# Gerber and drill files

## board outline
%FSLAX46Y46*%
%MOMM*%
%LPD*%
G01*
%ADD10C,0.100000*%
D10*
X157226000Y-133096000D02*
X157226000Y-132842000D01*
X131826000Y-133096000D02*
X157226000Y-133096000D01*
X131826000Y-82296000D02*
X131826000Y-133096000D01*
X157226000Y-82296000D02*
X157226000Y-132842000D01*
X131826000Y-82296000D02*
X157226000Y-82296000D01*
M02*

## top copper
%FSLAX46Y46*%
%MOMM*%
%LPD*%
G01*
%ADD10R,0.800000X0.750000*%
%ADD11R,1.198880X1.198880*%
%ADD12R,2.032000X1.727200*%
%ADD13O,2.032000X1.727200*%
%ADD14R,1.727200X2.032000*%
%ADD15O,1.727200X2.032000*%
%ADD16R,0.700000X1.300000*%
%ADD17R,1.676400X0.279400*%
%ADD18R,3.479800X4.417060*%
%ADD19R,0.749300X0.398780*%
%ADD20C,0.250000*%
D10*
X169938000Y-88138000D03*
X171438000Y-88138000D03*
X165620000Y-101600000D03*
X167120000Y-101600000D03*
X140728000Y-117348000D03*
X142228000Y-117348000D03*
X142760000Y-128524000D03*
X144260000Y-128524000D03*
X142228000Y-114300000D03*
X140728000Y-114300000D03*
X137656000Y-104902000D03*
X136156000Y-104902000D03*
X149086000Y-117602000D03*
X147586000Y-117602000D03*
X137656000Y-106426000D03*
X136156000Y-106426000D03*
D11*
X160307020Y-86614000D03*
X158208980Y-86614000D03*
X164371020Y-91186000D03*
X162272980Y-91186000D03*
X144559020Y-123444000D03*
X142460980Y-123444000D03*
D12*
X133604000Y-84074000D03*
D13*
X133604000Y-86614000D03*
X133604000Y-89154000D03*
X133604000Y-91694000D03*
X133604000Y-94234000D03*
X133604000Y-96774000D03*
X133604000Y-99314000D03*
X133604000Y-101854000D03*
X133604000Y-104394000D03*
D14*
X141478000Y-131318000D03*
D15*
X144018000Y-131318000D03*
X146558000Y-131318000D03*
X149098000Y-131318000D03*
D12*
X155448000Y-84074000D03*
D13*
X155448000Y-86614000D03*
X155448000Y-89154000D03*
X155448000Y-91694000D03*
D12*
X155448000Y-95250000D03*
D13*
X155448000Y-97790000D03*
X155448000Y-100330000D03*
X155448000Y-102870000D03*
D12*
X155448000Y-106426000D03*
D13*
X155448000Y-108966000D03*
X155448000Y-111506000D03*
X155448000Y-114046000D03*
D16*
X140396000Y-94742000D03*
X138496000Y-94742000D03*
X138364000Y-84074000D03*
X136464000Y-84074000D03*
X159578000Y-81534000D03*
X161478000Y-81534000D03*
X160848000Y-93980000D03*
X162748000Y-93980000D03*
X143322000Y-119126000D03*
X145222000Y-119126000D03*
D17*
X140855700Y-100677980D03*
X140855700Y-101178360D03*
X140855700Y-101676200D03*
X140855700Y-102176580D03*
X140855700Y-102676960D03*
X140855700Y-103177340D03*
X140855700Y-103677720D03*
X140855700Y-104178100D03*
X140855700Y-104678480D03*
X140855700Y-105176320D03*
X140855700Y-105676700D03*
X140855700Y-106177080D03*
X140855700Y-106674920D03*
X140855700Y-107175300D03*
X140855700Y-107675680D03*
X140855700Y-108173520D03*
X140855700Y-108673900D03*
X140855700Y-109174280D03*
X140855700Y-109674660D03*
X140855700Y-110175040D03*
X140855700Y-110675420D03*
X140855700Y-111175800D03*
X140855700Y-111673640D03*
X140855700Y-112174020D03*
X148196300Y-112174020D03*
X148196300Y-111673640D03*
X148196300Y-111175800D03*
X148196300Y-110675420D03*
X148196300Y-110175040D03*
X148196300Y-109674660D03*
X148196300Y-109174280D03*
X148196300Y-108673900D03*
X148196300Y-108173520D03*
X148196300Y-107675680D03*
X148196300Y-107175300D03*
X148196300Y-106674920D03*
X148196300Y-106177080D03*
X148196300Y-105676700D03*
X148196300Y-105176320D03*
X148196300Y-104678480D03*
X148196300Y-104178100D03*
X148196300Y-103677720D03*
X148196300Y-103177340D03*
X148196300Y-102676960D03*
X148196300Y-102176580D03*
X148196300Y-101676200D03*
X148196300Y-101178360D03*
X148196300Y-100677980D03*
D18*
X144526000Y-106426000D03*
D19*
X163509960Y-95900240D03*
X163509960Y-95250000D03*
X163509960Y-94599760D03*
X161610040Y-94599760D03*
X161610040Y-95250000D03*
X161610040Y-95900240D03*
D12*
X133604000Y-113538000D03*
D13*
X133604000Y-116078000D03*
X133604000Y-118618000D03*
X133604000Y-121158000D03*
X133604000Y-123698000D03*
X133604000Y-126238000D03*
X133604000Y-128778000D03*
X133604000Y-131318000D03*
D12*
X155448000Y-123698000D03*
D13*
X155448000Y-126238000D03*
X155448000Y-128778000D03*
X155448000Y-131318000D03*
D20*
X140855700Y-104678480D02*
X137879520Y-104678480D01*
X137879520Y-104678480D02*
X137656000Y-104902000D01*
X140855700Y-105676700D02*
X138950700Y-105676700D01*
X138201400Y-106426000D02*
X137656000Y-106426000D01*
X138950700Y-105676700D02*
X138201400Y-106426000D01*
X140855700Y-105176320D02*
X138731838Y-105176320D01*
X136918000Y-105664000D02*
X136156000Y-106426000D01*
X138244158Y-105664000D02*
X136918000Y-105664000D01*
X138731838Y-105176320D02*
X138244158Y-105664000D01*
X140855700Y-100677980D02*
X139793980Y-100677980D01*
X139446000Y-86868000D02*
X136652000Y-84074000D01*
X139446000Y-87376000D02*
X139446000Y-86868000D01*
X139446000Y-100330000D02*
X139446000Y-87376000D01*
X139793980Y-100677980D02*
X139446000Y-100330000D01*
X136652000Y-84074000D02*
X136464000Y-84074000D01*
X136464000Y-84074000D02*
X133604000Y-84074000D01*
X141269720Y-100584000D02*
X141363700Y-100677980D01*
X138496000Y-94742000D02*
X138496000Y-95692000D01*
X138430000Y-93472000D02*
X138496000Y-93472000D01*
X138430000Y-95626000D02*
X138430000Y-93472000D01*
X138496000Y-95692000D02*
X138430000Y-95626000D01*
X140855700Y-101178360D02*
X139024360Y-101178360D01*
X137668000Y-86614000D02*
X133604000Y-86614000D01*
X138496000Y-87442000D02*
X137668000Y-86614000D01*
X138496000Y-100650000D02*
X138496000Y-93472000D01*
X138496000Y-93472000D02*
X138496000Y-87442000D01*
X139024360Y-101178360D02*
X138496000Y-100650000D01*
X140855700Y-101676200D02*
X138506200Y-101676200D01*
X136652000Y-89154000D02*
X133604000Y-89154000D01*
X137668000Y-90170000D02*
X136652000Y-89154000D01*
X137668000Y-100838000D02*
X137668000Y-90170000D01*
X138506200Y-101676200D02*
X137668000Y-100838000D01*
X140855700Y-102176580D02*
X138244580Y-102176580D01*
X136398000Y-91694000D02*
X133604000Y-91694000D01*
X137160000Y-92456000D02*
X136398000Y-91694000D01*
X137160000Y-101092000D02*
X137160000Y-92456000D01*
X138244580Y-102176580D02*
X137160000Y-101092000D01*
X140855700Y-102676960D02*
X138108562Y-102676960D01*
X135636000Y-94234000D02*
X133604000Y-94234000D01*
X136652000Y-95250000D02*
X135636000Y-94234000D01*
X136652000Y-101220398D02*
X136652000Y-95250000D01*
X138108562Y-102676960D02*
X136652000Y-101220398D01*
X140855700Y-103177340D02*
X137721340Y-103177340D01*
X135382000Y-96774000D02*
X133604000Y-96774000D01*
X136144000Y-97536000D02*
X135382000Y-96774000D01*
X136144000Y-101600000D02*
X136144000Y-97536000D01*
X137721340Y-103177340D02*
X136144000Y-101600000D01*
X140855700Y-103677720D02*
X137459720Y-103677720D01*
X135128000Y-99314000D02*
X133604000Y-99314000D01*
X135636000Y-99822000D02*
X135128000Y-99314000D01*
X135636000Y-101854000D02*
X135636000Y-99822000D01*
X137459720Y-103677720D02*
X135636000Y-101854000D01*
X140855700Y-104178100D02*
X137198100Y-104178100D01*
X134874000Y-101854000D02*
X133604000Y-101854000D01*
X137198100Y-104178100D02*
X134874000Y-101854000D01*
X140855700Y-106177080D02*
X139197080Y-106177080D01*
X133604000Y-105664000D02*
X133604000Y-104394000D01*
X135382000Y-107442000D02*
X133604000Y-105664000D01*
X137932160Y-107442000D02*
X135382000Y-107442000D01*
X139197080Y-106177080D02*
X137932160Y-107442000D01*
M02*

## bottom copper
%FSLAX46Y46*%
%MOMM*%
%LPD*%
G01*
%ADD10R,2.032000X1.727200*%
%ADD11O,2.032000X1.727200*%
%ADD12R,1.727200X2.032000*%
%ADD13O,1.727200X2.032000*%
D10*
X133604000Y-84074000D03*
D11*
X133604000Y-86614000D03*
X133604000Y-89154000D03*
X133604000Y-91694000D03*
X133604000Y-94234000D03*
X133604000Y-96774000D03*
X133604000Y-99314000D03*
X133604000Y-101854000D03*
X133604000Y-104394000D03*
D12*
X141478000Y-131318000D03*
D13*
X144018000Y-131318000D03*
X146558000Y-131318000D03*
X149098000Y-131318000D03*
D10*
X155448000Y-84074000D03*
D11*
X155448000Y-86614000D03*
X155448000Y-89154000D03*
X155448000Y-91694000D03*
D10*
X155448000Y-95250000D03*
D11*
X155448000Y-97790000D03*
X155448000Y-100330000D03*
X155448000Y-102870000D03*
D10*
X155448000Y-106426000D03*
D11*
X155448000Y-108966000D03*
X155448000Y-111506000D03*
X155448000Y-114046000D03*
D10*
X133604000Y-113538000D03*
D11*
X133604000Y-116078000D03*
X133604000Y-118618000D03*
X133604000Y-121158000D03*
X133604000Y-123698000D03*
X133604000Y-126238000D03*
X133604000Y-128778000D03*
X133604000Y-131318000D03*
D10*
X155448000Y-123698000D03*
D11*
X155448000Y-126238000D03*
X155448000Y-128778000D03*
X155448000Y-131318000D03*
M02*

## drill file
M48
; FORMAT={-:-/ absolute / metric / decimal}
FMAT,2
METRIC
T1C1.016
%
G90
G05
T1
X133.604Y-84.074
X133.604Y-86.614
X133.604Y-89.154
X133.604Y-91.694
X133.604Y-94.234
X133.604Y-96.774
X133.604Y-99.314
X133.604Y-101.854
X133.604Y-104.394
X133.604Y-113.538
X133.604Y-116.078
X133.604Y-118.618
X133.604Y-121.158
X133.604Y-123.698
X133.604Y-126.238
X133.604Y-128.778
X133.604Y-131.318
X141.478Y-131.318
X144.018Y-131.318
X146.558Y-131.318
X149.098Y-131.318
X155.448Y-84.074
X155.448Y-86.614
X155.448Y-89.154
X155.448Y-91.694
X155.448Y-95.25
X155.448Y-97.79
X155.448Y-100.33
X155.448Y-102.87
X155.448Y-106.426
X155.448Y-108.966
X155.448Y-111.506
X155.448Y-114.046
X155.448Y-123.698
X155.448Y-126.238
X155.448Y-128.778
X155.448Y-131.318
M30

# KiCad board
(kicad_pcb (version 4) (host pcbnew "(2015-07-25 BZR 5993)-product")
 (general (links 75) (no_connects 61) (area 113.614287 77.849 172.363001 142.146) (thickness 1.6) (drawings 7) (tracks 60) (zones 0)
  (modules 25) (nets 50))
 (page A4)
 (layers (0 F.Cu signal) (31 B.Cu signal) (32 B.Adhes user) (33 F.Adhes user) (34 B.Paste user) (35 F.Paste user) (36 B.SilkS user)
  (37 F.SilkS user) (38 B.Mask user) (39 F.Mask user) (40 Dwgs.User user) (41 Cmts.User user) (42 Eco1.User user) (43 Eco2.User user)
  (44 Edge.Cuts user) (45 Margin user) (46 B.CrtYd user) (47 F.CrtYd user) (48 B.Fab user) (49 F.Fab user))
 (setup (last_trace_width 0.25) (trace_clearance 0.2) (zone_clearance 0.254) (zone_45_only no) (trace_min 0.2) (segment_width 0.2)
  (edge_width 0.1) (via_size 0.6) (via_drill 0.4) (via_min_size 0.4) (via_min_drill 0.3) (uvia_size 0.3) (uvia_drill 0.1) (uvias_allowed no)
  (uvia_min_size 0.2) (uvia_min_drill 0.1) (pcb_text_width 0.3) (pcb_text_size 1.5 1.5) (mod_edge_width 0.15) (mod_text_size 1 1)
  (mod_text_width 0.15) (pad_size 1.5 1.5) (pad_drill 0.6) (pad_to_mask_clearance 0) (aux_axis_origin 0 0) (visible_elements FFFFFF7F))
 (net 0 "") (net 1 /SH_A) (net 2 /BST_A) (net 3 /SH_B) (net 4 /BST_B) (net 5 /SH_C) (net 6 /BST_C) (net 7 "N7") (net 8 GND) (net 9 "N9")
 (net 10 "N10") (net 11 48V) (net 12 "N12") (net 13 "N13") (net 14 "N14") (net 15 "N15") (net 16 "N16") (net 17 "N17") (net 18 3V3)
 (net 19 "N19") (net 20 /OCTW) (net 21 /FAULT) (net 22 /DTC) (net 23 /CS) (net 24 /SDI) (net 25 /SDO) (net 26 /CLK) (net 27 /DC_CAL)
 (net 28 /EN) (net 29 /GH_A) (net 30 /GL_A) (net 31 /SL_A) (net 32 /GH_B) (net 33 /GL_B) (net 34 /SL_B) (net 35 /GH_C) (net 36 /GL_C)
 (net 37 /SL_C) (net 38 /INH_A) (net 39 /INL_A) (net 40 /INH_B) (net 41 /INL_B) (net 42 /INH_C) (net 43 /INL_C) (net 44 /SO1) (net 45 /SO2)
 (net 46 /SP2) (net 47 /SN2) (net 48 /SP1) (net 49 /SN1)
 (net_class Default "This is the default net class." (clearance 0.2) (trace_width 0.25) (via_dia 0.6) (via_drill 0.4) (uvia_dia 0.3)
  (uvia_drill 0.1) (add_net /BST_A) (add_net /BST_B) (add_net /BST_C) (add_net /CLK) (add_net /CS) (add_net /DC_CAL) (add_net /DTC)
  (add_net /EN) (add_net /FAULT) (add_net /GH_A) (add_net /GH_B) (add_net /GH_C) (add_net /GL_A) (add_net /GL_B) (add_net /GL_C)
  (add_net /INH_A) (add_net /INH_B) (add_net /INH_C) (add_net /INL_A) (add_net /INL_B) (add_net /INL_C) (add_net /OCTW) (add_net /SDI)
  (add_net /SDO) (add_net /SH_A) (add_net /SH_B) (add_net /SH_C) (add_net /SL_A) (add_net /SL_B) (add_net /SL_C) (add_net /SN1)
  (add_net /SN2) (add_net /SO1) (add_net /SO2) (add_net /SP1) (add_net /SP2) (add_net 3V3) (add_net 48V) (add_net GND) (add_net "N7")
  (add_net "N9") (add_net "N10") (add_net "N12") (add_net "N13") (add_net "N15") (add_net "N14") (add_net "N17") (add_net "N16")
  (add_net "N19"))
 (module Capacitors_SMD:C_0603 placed (layer F.Cu) (at 170.688 88.138)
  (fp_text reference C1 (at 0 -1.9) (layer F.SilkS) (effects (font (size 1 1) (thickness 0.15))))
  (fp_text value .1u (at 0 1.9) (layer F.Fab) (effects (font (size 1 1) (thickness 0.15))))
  (pad 1 smd rect (at -0.75 0) (size 0.8 0.75) (layers F.Cu F.Paste F.Mask) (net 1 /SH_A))
  (pad 2 smd rect (at 0.75 0) (size 0.8 0.75) (layers F.Cu F.Paste F.Mask) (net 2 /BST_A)))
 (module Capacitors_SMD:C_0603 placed (layer F.Cu) (at 166.37 101.6)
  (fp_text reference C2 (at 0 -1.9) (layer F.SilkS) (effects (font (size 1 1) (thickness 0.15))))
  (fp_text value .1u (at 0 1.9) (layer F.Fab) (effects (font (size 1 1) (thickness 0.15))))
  (pad 1 smd rect (at -0.75 0) (size 0.8 0.75) (layers F.Cu F.Paste F.Mask) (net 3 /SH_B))
  (pad 2 smd rect (at 0.75 0) (size 0.8 0.75) (layers F.Cu F.Paste F.Mask) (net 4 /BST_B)))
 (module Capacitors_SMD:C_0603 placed (layer F.Cu) (at 141.478 117.348)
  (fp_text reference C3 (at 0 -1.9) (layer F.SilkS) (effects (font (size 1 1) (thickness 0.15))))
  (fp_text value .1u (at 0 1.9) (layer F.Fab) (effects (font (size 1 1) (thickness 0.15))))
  (pad 1 smd rect (at -0.75 0) (size 0.8 0.75) (layers F.Cu F.Paste F.Mask) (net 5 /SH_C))
  (pad 2 smd rect (at 0.75 0) (size 0.8 0.75) (layers F.Cu F.Paste F.Mask) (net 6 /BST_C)))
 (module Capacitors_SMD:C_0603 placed (layer F.Cu) (at 143.51 128.524)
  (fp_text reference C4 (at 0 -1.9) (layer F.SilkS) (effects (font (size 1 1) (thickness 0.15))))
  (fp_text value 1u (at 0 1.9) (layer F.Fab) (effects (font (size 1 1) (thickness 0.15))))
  (pad 1 smd rect (at -0.75 0) (size 0.8 0.75) (layers F.Cu F.Paste F.Mask) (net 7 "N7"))
  (pad 2 smd rect (at 0.75 0) (size 0.8 0.75) (layers F.Cu F.Paste F.Mask) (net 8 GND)))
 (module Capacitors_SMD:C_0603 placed (layer F.Cu) (at 141.478 114.3 180)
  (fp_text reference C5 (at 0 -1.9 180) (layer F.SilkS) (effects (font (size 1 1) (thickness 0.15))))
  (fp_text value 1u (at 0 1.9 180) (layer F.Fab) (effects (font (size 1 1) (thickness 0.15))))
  (pad 1 smd rect (at -0.75 0 180) (size 0.8 0.75) (layers F.Cu F.Paste F.Mask) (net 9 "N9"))
  (pad 2 smd rect (at 0.75 0 180) (size 0.8 0.75) (layers F.Cu F.Paste F.Mask) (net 8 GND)))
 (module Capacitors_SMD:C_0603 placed (layer F.Cu) (at 136.906 104.902 180)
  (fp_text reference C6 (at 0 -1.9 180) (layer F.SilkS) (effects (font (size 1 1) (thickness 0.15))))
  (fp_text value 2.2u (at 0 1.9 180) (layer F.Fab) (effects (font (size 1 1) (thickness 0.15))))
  (pad 1 smd rect (at -0.75 0 180) (size 0.8 0.75) (layers F.Cu F.Paste F.Mask) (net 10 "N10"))
  (pad 2 smd rect (at 0.75 0 180) (size 0.8 0.75) (layers F.Cu F.Paste F.Mask) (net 8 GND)))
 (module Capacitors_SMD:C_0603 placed (layer F.Cu) (at 148.336 117.602 180)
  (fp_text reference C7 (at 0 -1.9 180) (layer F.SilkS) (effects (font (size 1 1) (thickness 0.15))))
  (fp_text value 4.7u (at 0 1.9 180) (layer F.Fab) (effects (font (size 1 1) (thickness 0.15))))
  (pad 1 smd rect (at -0.75 0 180) (size 0.8 0.75) (layers F.Cu F.Paste F.Mask) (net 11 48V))
  (pad 2 smd rect (at 0.75 0 180) (size 0.8 0.75) (layers F.Cu F.Paste F.Mask) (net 8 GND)))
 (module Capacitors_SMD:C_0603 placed (layer F.Cu) (at 136.906 106.426 180)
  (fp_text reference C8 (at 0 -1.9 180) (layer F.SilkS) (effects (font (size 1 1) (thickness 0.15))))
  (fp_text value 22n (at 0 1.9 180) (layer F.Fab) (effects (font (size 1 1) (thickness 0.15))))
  (pad 1 smd rect (at -0.75 0 180) (size 0.8 0.75) (layers F.Cu F.Paste F.Mask) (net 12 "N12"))
  (pad 2 smd rect (at 0.75 0 180) (size 0.8 0.75) (layers F.Cu F.Paste F.Mask) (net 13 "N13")))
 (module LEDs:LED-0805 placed (layer F.Cu) (at 159.258 86.614)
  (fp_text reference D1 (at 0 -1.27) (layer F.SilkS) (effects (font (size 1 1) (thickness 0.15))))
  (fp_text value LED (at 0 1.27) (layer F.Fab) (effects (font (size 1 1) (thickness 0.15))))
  (pad 2 smd rect (at 1.04902 0 180) (size 1.19888 1.19888) (layers F.Cu F.Paste F.Mask) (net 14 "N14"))
  (pad 1 smd rect (at -1.04902 0 180) (size 1.19888 1.19888) (layers F.Cu F.Paste F.Mask) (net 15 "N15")))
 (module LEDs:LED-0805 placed (layer F.Cu) (at 163.322 91.186)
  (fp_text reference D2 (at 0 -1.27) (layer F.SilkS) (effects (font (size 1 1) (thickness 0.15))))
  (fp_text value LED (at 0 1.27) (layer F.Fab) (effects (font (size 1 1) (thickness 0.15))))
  (pad 2 smd rect (at 1.04902 0 180) (size 1.19888 1.19888) (layers F.Cu F.Paste F.Mask) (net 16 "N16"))
  (pad 1 smd rect (at -1.04902 0 180) (size 1.19888 1.19888) (layers F.Cu F.Paste F.Mask) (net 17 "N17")))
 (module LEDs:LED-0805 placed (layer F.Cu) (at 143.51 123.444)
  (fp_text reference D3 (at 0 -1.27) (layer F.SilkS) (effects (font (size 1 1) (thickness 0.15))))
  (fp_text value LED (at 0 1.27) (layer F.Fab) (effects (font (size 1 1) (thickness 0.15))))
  (pad 2 smd rect (at 1.04902 0 180) (size 1.19888 1.19888) (layers F.Cu F.Paste F.Mask) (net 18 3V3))
  (pad 1 smd rect (at -1.04902 0 180) (size 1.19888 1.19888) (layers F.Cu F.Paste F.Mask) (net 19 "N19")))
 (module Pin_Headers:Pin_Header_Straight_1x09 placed (layer F.Cu) (at 133.604 84.074)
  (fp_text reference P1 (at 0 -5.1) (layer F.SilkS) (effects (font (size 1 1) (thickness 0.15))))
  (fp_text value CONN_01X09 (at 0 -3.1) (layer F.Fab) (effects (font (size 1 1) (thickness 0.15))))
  (pad 1 thru_hole rect (at 0 0) (size 2.032 1.7272) (drill 1.016) (layers *.Cu *.Mask F.SilkS) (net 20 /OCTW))
  (pad 2 thru_hole oval (at 0 2.54) (size 2.032 1.7272) (drill 1.016) (layers *.Cu *.Mask F.SilkS) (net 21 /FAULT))
  (pad 3 thru_hole oval (at 0 5.08) (size 2.032 1.7272) (drill 1.016) (layers *.Cu *.Mask F.SilkS) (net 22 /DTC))
  (pad 4 thru_hole oval (at 0 7.62) (size 2.032 1.7272) (drill 1.016) (layers *.Cu *.Mask F.SilkS) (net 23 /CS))
  (pad 5 thru_hole oval (at 0 10.16) (size 2.032 1.7272) (drill 1.016) (layers *.Cu *.Mask F.SilkS) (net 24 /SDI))
  (pad 6 thru_hole oval (at 0 12.7) (size 2.032 1.7272) (drill 1.016) (layers *.Cu *.Mask F.SilkS) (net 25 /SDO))
  (pad 7 thru_hole oval (at 0 15.24) (size 2.032 1.7272) (drill 1.016) (layers *.Cu *.Mask F.SilkS) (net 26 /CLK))
  (pad 8 thru_hole oval (at 0 17.78) (size 2.032 1.7272) (drill 1.016) (layers *.Cu *.Mask F.SilkS) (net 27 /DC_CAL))
  (pad 9 thru_hole oval (at 0 20.32) (size 2.032 1.7272) (drill 1.016) (layers *.Cu *.Mask F.SilkS) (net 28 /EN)))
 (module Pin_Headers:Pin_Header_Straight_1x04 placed (layer F.Cu) (at 141.478 131.318 90)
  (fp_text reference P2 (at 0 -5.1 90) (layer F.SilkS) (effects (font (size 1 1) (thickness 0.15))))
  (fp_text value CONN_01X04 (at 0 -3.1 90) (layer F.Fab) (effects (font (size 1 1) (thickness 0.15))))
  (pad 1 thru_hole rect (at 0 0 90) (size 2.032 1.7272) (drill 1.016) (layers *.Cu *.Mask F.SilkS) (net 18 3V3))
  (pad 2 thru_hole oval (at 0 2.54 90) (size 2.032 1.7272) (drill 1.016) (layers *.Cu *.Mask F.SilkS) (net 11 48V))
  (pad 3 thru_hole oval (at 0 5.08 90) (size 2.032 1.7272) (drill 1.016) (layers *.Cu *.Mask F.SilkS) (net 8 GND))
  (pad 4 thru_hole oval (at 0 7.62 90) (size 2.032 1.7272) (drill 1.016) (layers *.Cu *.Mask F.SilkS) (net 8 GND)))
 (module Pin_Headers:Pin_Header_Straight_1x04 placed (layer F.Cu) (at 155.448 84.074)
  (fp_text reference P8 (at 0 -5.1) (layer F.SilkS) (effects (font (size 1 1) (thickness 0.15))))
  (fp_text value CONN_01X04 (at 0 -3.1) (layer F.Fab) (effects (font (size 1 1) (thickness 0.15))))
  (pad 1 thru_hole rect (at 0 0) (size 2.032 1.7272) (drill 1.016) (layers *.Cu *.Mask F.SilkS) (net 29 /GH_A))
  (pad 2 thru_hole oval (at 0 2.54) (size 2.032 1.7272) (drill 1.016) (layers *.Cu *.Mask F.SilkS) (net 1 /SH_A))
  (pad 3 thru_hole oval (at 0 5.08) (size 2.032 1.7272) (drill 1.016) (layers *.Cu *.Mask F.SilkS) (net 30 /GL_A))
  (pad 4 thru_hole oval (at 0 7.62) (size 2.032 1.7272) (drill 1.016) (layers *.Cu *.Mask F.SilkS) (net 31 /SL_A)))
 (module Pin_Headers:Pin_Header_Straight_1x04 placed (layer F.Cu) (at 155.448 95.25)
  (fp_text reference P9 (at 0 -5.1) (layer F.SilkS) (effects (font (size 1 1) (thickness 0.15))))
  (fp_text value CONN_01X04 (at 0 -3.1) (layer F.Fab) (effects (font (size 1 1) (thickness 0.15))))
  (pad 1 thru_hole rect (at 0 0) (size 2.032 1.7272) (drill 1.016) (layers *.Cu *.Mask F.SilkS) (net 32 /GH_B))
  (pad 2 thru_hole oval (at 0 2.54) (size 2.032 1.7272) (drill 1.016) (layers *.Cu *.Mask F.SilkS) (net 3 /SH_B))
  (pad 3 thru_hole oval (at 0 5.08) (size 2.032 1.7272) (drill 1.016) (layers *.Cu *.Mask F.SilkS) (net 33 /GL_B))
  (pad 4 thru_hole oval (at 0 7.62) (size 2.032 1.7272) (drill 1.016) (layers *.Cu *.Mask F.SilkS) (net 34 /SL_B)))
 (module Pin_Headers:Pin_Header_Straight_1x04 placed (layer F.Cu) (at 155.448 106.426)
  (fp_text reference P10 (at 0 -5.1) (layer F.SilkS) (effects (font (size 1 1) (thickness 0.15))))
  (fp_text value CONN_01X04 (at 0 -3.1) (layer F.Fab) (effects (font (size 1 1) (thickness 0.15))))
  (pad 1 thru_hole rect (at 0 0) (size 2.032 1.7272) (drill 1.016) (layers *.Cu *.Mask F.SilkS) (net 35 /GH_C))
  (pad 2 thru_hole oval (at 0 2.54) (size 2.032 1.7272) (drill 1.016) (layers *.Cu *.Mask F.SilkS) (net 5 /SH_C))
  (pad 3 thru_hole oval (at 0 5.08) (size 2.032 1.7272) (drill 1.016) (layers *.Cu *.Mask F.SilkS) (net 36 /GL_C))
  (pad 4 thru_hole oval (at 0 7.62) (size 2.032 1.7272) (drill 1.016) (layers *.Cu *.Mask F.SilkS) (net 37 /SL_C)))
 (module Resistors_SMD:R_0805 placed (layer F.Cu) (at 139.446 94.742 180)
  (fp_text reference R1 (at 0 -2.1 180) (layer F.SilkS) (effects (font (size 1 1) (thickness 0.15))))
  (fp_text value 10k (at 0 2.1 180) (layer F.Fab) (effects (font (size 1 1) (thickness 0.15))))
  (pad 1 smd rect (at -0.95 0 180) (size 0.7 1.3) (layers F.Cu F.Paste F.Mask) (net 18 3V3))
  (pad 2 smd rect (at 0.95 0 180) (size 0.7 1.3) (layers F.Cu F.Paste F.Mask) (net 21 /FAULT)))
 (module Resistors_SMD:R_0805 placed (layer F.Cu) (at 137.414 84.074 180)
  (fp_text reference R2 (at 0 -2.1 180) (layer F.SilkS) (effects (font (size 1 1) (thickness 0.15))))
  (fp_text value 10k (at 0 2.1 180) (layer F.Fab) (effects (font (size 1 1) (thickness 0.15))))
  (pad 1 smd rect (at -0.95 0 180) (size 0.7 1.3) (layers F.Cu F.Paste F.Mask) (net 18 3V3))
  (pad 2 smd rect (at 0.95 0 180) (size 0.7 1.3) (layers F.Cu F.Paste F.Mask) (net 20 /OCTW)))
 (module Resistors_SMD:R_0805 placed (layer F.Cu) (at 160.528 81.534)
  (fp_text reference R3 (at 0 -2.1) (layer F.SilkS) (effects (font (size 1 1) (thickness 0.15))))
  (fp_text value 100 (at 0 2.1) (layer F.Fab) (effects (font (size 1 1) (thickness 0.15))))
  (pad 1 smd rect (at -0.95 0) (size 0.7 1.3) (layers F.Cu F.Paste F.Mask) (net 15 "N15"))
  (pad 2 smd rect (at 0.95 0) (size 0.7 1.3) (layers F.Cu F.Paste F.Mask) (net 8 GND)))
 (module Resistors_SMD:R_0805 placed (layer F.Cu) (at 161.798 93.98)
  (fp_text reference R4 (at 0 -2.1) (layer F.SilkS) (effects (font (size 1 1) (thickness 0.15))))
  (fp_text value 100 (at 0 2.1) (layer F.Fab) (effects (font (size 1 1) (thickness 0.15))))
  (pad 1 smd rect (at -0.95 0) (size 0.7 1.3) (layers F.Cu F.Paste F.Mask) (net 17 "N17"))
  (pad 2 smd rect (at 0.95 0) (size 0.7 1.3) (layers F.Cu F.Paste F.Mask) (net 8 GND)))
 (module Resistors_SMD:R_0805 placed (layer F.Cu) (at 144.272 119.126)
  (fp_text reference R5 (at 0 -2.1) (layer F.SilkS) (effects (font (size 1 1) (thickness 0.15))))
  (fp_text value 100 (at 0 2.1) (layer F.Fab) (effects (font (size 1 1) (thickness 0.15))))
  (pad 1 smd rect (at -0.95 0) (size 0.7 1.3) (layers F.Cu F.Paste F.Mask) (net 19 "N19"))
  (pad 2 smd rect (at 0.95 0) (size 0.7 1.3) (layers F.Cu F.Paste F.Mask) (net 8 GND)))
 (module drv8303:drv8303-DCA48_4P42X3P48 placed (layer F.Cu) (at 144.526 106.426)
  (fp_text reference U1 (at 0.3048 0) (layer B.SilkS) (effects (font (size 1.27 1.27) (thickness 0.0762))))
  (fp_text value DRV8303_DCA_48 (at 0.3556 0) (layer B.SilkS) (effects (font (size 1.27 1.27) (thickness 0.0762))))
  (pad 1 smd rect (at -3.6703 -5.74802) (size 1.6764 0.2794) (layers F.Cu F.Paste F.Mask) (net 20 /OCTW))
  (pad 2 smd rect (at -3.6703 -5.24764) (size 1.6764 0.2794) (layers F.Cu F.Paste F.Mask) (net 21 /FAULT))
  (pad 3 smd rect (at -3.6703 -4.7498) (size 1.6764 0.2794) (layers F.Cu F.Paste F.Mask) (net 22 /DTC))
  (pad 4 smd rect (at -3.6703 -4.24942) (size 1.6764 0.2794) (layers F.Cu F.Paste F.Mask) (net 23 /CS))
  (pad 5 smd rect (at -3.6703 -3.74904) (size 1.6764 0.2794) (layers F.Cu F.Paste F.Mask) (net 24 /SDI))
  (pad 6 smd rect (at -3.6703 -3.24866) (size 1.6764 0.2794) (layers F.Cu F.Paste F.Mask) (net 25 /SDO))
  (pad 7 smd rect (at -3.6703 -2.74828) (size 1.6764 0.2794) (layers F.Cu F.Paste F.Mask) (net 26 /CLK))
  (pad 8 smd rect (at -3.6703 -2.2479) (size 1.6764 0.2794) (layers F.Cu F.Paste F.Mask) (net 27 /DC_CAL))
  (pad 9 smd rect (at -3.6703 -1.74752) (size 1.6764 0.2794) (layers F.Cu F.Paste F.Mask) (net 10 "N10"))
  (pad 10 smd rect (at -3.6703 -1.24968) (size 1.6764 0.2794) (layers F.Cu F.Paste F.Mask) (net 13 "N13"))
  (pad 11 smd rect (at -3.6703 -0.7493) (size 1.6764 0.2794) (layers F.Cu F.Paste F.Mask) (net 12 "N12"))
  (pad 12 smd rect (at -3.6703 -0.24892) (size 1.6764 0.2794) (layers F.Cu F.Paste F.Mask) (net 28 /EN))
  (pad 13 smd rect (at -3.6703 0.24892) (size 1.6764 0.2794) (layers F.Cu F.Paste F.Mask) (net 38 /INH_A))
  (pad 14 smd rect (at -3.6703 0.7493) (size 1.6764 0.2794) (layers F.Cu F.Paste F.Mask) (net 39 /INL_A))
  (pad 15 smd rect (at -3.6703 1.24968) (size 1.6764 0.2794) (layers F.Cu F.Paste F.Mask) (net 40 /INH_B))
  (pad 16 smd rect (at -3.6703 1.74752) (size 1.6764 0.2794) (layers F.Cu F.Paste F.Mask) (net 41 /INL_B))
  (pad 17 smd rect (at -3.6703 2.2479) (size 1.6764 0.2794) (layers F.Cu F.Paste F.Mask) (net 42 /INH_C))
  (pad 18 smd rect (at -3.6703 2.74828) (size 1.6764 0.2794) (layers F.Cu F.Paste F.Mask) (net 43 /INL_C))
  (pad 19 smd rect (at -3.6703 3.24866) (size 1.6764 0.2794) (layers F.Cu F.Paste F.Mask) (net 9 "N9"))
  (pad 20 smd rect (at -3.6703 3.74904) (size 1.6764 0.2794) (layers F.Cu F.Paste F.Mask) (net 18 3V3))
  (pad 21 smd rect (at -3.6703 4.24942) (size 1.6764 0.2794) (layers F.Cu F.Paste F.Mask) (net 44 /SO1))
  (pad 22 smd rect (at -3.6703 4.7498) (size 1.6764 0.2794) (layers F.Cu F.Paste F.Mask) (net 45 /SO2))
  (pad 23 smd rect (at -3.6703 5.24764) (size 1.6764 0.2794) (layers F.Cu F.Paste F.Mask) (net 7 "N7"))
  (pad 24 smd rect (at -3.6703 5.74802) (size 1.6764 0.2794) (layers F.Cu F.Paste F.Mask) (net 8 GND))
  (pad 25 smd rect (at 3.6703 5.74802) (size 1.6764 0.2794) (layers F.Cu F.Paste F.Mask) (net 11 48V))
  (pad 26 smd rect (at 3.6703 5.24764) (size 1.6764 0.2794) (layers F.Cu F.Paste F.Mask) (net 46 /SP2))
  (pad 27 smd rect (at 3.6703 4.7498) (size 1.6764 0.2794) (layers F.Cu F.Paste F.Mask) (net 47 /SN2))
  (pad 28 smd rect (at 3.6703 4.24942) (size 1.6764 0.2794) (layers F.Cu F.Paste F.Mask) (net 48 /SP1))
  (pad 29 smd rect (at 3.6703 3.74904) (size 1.6764 0.2794) (layers F.Cu F.Paste F.Mask) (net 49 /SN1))
  (pad 30 smd rect (at 3.6703 3.24866) (size 1.6764 0.2794) (layers F.Cu F.Paste F.Mask) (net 37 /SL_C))
  (pad 31 smd rect (at 3.6703 2.74828) (size 1.6764 0.2794) (layers F.Cu F.Paste F.Mask) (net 36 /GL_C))
  (pad 32 smd rect (at 3.6703 2.2479) (size 1.6764 0.2794) (layers F.Cu F.Paste F.Mask) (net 5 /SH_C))
  (pad 33 smd rect (at 3.6703 1.74752) (size 1.6764 0.2794) (layers F.Cu F.Paste F.Mask) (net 35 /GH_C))
  (pad 34 smd rect (at 3.6703 1.24968) (size 1.6764 0.2794) (layers F.Cu F.Paste F.Mask) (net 6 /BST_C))
  (pad 35 smd rect (at 3.6703 0.7493) (size 1.6764 0.2794) (layers F.Cu F.Paste F.Mask) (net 34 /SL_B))
  (pad 36 smd rect (at 3.6703 0.24892) (size 1.6764 0.2794) (layers F.Cu F.Paste F.Mask) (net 33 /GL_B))
  (pad 37 smd rect (at 3.6703 -0.24892) (size 1.6764 0.2794) (layers F.Cu F.Paste F.Mask) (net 3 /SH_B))
  (pad 38 smd rect (at 3.6703 -0.7493) (size 1.6764 0.2794) (layers F.Cu F.Paste F.Mask) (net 32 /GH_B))
  (pad 39 smd rect (at 3.6703 -1.24968) (size 1.6764 0.2794) (layers F.Cu F.Paste F.Mask) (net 4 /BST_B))
  (pad 40 smd rect (at 3.6703 -1.74752) (size 1.6764 0.2794) (layers F.Cu F.Paste F.Mask) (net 31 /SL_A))
  (pad 41 smd rect (at 3.6703 -2.2479) (size 1.6764 0.2794) (layers F.Cu F.Paste F.Mask) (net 30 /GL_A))
  (pad 42 smd rect (at 3.6703 -2.74828) (size 1.6764 0.2794) (layers F.Cu F.Paste F.Mask) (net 1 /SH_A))
  (pad 43 smd rect (at 3.6703 -3.24866) (size 1.6764 0.2794) (layers F.Cu F.Paste F.Mask) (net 29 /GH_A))
  (pad 44 smd rect (at 3.6703 -3.74904) (size 1.6764 0.2794) (layers F.Cu F.Paste F.Mask) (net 2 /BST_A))
  (pad 45 smd rect (at 3.6703 -4.24942) (size 1.6764 0.2794) (layers F.Cu F.Paste F.Mask) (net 18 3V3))
  (pad 46 smd rect (at 3.6703 -4.7498) (size 1.6764 0.2794) (layers F.Cu F.Paste F.Mask) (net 8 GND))
  (pad 47 smd rect (at 3.6703 -5.24764) (size 1.6764 0.2794) (layers F.Cu F.Paste F.Mask) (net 8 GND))
  (pad 48 smd rect (at 3.6703 -5.74802) (size 1.6764 0.2794) (layers F.Cu F.Paste F.Mask) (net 8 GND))
  (pad 49 smd rect (at 0 0) (size 3.4798 4.41706) (layers F.Cu F.Paste F.Mask) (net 8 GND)))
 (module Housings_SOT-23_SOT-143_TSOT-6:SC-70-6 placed (layer F.Cu) (at 162.56 95.25 90)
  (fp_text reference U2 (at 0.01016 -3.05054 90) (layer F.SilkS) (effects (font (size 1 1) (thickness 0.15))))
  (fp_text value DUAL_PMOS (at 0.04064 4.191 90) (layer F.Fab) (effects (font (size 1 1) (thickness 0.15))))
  (pad 1 smd rect (at -0.65024 0.94996 90) (size 0.39878 0.7493) (layers F.Cu F.Paste F.Mask) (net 18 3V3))
  (pad 2 smd rect (at 0 0.94996 90) (size 0.39878 0.7493) (layers F.Cu F.Paste F.Mask) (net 20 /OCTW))
  (pad 3 smd rect (at 0.65024 0.94996 90) (size 0.39878 0.7493) (layers F.Cu F.Paste F.Mask) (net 14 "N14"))
  (pad 4 smd rect (at 0.65024 -0.94996 90) (size 0.39878 0.7493) (layers F.Cu F.Paste F.Mask) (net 18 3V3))
  (pad 5 smd rect (at 0 -0.94996 90) (size 0.39878 0.7493) (layers F.Cu F.Paste F.Mask) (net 21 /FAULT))
  (pad 6 smd rect (at -0.65024 -0.94996 90) (size 0.39878 0.7493) (layers F.Cu F.Paste F.Mask) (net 16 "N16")))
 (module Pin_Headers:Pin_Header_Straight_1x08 (layer F.Cu) (at 133.604 113.538)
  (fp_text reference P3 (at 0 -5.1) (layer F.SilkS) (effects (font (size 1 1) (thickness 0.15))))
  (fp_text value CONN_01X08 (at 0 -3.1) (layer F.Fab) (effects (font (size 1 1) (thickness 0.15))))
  (pad 1 thru_hole rect (at 0 0) (size 2.032 1.7272) (drill 1.016) (layers *.Cu *.Mask F.SilkS) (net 38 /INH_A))
  (pad 2 thru_hole oval (at 0 2.54) (size 2.032 1.7272) (drill 1.016) (layers *.Cu *.Mask F.SilkS) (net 39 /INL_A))
  (pad 3 thru_hole oval (at 0 5.08) (size 2.032 1.7272) (drill 1.016) (layers *.Cu *.Mask F.SilkS) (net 40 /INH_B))
  (pad 4 thru_hole oval (at 0 7.62) (size 2.032 1.7272) (drill 1.016) (layers *.Cu *.Mask F.SilkS) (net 41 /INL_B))
  (pad 5 thru_hole oval (at 0 10.16) (size 2.032 1.7272) (drill 1.016) (layers *.Cu *.Mask F.SilkS) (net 42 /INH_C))
  (pad 6 thru_hole oval (at 0 12.7) (size 2.032 1.7272) (drill 1.016) (layers *.Cu *.Mask F.SilkS) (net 43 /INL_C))
  (pad 7 thru_hole oval (at 0 15.24) (size 2.032 1.7272) (drill 1.016) (layers *.Cu *.Mask F.SilkS) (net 44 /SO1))
  (pad 8 thru_hole oval (at 0 17.78) (size 2.032 1.7272) (drill 1.016) (layers *.Cu *.Mask F.SilkS) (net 45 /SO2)))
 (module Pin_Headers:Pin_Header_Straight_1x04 (layer F.Cu) (at 155.448 123.698)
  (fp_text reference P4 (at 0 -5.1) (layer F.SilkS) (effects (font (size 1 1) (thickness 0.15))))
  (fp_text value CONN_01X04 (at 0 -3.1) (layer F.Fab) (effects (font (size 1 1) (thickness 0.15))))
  (pad 1 thru_hole rect (at 0 0) (size 2.032 1.7272) (drill 1.016) (layers *.Cu *.Mask F.SilkS) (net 49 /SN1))
  (pad 2 thru_hole oval (at 0 2.54) (size 2.032 1.7272) (drill 1.016) (layers *.Cu *.Mask F.SilkS) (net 48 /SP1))
  (pad 3 thru_hole oval (at 0 5.08) (size 2.032 1.7272) (drill 1.016) (layers *.Cu *.Mask F.SilkS) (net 47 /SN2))
  (pad 4 thru_hole oval (at 0 7.62) (size 2.032 1.7272) (drill 1.016) (layers *.Cu *.Mask F.SilkS) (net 46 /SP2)))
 (gr_line (start 157.226 133.096) (end 157.226 132.842) (angle 90) (layer Edge.Cuts) (width 0.1))
 (gr_line (start 131.826 133.096) (end 157.226 133.096) (angle 90) (layer Edge.Cuts) (width 0.1))
 (gr_line (start 131.826 82.296) (end 131.826 133.096) (angle 90) (layer Edge.Cuts) (width 0.1))
 (gr_line (start 157.226 82.296) (end 157.226 132.842) (angle 90) (layer Edge.Cuts) (width 0.1))
 (gr_line (start 131.826 82.296) (end 157.226 82.296) (angle 90) (layer Edge.Cuts) (width 0.1))
 (segment (start 140.8557 104.67848) (end 137.87952 104.67848) (width 0.25) (layer F.Cu) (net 10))
 (segment (start 137.87952 104.67848) (end 137.656 104.902) (width 0.25) (layer F.Cu) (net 10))
 (segment (start 140.8557 105.6767) (end 138.9507 105.6767) (width 0.25) (layer F.Cu) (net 12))
 (segment (start 138.2014 106.426) (end 137.656 106.426) (width 0.25) (layer F.Cu) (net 12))
 (segment (start 138.9507 105.6767) (end 138.2014 106.426) (width 0.25) (layer F.Cu) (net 12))
 (segment (start 140.8557 105.17632) (end 138.731838 105.17632) (width 0.25) (layer F.Cu) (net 13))
 (segment (start 136.918 105.664) (end 136.156 106.426) (width 0.25) (layer F.Cu) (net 13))
 (segment (start 138.244158 105.664) (end 136.918 105.664) (width 0.25) (layer F.Cu) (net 13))
 (segment (start 138.731838 105.17632) (end 138.244158 105.664) (width 0.25) (layer F.Cu) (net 13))
 (segment (start 140.8557 100.67798) (end 139.79398 100.67798) (width 0.25) (layer F.Cu) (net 20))
 (segment (start 139.446 86.868) (end 136.652 84.074) (width 0.25) (layer F.Cu) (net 20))
 (segment (start 139.446 87.376) (end 139.446 86.868) (width 0.25) (layer F.Cu) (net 20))
 (segment (start 139.446 100.33) (end 139.446 87.376) (width 0.25) (layer F.Cu) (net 20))
 (segment (start 139.79398 100.67798) (end 139.446 100.33) (width 0.25) (layer F.Cu) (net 20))
 (segment (start 136.652 84.074) (end 136.464 84.074) (width 0.25) (layer F.Cu) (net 20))
 (segment (start 136.464 84.074) (end 133.604 84.074) (width 0.25) (layer F.Cu) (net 20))
 (segment (start 141.26972 100.584) (end 141.3637 100.67798) (width 0.25) (layer F.Cu) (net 20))
 (segment (start 138.496 94.742) (end 138.496 95.692) (width 0.25) (layer F.Cu) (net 21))
 (segment (start 138.43 93.472) (end 138.496 93.472) (width 0.25) (layer F.Cu) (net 21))
 (segment (start 138.43 95.626) (end 138.43 93.472) (width 0.25) (layer F.Cu) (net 21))
 (segment (start 138.496 95.692) (end 138.43 95.626) (width 0.25) (layer F.Cu) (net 21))
 (segment (start 140.8557 101.17836) (end 139.02436 101.17836) (width 0.25) (layer F.Cu) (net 21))
 (segment (start 137.668 86.614) (end 133.604 86.614) (width 0.25) (layer F.Cu) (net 21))
 (segment (start 138.496 87.442) (end 137.668 86.614) (width 0.25) (layer F.Cu) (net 21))
 (segment (start 138.496 100.65) (end 138.496 93.472) (width 0.25) (layer F.Cu) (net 21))
 (segment (start 138.496 93.472) (end 138.496 87.442) (width 0.25) (layer F.Cu) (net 21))
 (segment (start 139.02436 101.17836) (end 138.496 100.65) (width 0.25) (layer F.Cu) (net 21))
 (segment (start 140.8557 101.6762) (end 138.5062 101.6762) (width 0.25) (layer F.Cu) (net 22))
 (segment (start 136.652 89.154) (end 133.604 89.154) (width 0.25) (layer F.Cu) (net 22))
 (segment (start 137.668 90.17) (end 136.652 89.154) (width 0.25) (layer F.Cu) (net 22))
 (segment (start 137.668 100.838) (end 137.668 90.17) (width 0.25) (layer F.Cu) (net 22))
 (segment (start 138.5062 101.6762) (end 137.668 100.838) (width 0.25) (layer F.Cu) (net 22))
 (segment (start 140.8557 102.17658) (end 138.24458 102.17658) (width 0.25) (layer F.Cu) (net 23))
 (segment (start 136.398 91.694) (end 133.604 91.694) (width 0.25) (layer F.Cu) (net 23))
 (segment (start 137.16 92.456) (end 136.398 91.694) (width 0.25) (layer F.Cu) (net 23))
 (segment (start 137.16 101.092) (end 137.16 92.456) (width 0.25) (layer F.Cu) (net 23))
 (segment (start 138.24458 102.17658) (end 137.16 101.092) (width 0.25) (layer F.Cu) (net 23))
 (segment (start 140.8557 102.67696) (end 138.108562 102.67696) (width 0.25) (layer F.Cu) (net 24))
 (segment (start 135.636 94.234) (end 133.604 94.234) (width 0.25) (layer F.Cu) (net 24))
 (segment (start 136.652 95.25) (end 135.636 94.234) (width 0.25) (layer F.Cu) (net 24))
 (segment (start 136.652 101.220398) (end 136.652 95.25) (width 0.25) (layer F.Cu) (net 24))
 (segment (start 138.108562 102.67696) (end 136.652 101.220398) (width 0.25) (layer F.Cu) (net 24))
 (segment (start 140.8557 103.17734) (end 137.72134 103.17734) (width 0.25) (layer F.Cu) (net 25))
 (segment (start 135.382 96.774) (end 133.604 96.774) (width 0.25) (layer F.Cu) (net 25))
 (segment (start 136.144 97.536) (end 135.382 96.774) (width 0.25) (layer F.Cu) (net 25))
 (segment (start 136.144 101.6) (end 136.144 97.536) (width 0.25) (layer F.Cu) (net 25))
 (segment (start 137.72134 103.17734) (end 136.144 101.6) (width 0.25) (layer F.Cu) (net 25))
 (segment (start 140.8557 103.67772) (end 137.45972 103.67772) (width 0.25) (layer F.Cu) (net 26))
 (segment (start 135.128 99.314) (end 133.604 99.314) (width 0.25) (layer F.Cu) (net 26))
 (segment (start 135.636 99.822) (end 135.128 99.314) (width 0.25) (layer F.Cu) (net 26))
 (segment (start 135.636 101.854) (end 135.636 99.822) (width 0.25) (layer F.Cu) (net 26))
 (segment (start 137.45972 103.67772) (end 135.636 101.854) (width 0.25) (layer F.Cu) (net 26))
 (segment (start 140.8557 104.1781) (end 137.1981 104.1781) (width 0.25) (layer F.Cu) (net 27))
 (segment (start 134.874 101.854) (end 133.604 101.854) (width 0.25) (layer F.Cu) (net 27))
 (segment (start 137.1981 104.1781) (end 134.874 101.854) (width 0.25) (layer F.Cu) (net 27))
 (segment (start 140.8557 106.17708) (end 139.19708 106.17708) (width 0.25) (layer F.Cu) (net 28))
 (segment (start 133.604 105.664) (end 133.604 104.394) (width 0.25) (layer F.Cu) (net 28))
 (segment (start 135.382 107.442) (end 133.604 105.664) (width 0.25) (layer F.Cu) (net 28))
 (segment (start 137.93216 107.442) (end 135.382 107.442) (width 0.25) (layer F.Cu) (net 28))
 (segment (start 139.19708 106.17708) (end 137.93216 107.442) (width 0.25) (layer F.Cu) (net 28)))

